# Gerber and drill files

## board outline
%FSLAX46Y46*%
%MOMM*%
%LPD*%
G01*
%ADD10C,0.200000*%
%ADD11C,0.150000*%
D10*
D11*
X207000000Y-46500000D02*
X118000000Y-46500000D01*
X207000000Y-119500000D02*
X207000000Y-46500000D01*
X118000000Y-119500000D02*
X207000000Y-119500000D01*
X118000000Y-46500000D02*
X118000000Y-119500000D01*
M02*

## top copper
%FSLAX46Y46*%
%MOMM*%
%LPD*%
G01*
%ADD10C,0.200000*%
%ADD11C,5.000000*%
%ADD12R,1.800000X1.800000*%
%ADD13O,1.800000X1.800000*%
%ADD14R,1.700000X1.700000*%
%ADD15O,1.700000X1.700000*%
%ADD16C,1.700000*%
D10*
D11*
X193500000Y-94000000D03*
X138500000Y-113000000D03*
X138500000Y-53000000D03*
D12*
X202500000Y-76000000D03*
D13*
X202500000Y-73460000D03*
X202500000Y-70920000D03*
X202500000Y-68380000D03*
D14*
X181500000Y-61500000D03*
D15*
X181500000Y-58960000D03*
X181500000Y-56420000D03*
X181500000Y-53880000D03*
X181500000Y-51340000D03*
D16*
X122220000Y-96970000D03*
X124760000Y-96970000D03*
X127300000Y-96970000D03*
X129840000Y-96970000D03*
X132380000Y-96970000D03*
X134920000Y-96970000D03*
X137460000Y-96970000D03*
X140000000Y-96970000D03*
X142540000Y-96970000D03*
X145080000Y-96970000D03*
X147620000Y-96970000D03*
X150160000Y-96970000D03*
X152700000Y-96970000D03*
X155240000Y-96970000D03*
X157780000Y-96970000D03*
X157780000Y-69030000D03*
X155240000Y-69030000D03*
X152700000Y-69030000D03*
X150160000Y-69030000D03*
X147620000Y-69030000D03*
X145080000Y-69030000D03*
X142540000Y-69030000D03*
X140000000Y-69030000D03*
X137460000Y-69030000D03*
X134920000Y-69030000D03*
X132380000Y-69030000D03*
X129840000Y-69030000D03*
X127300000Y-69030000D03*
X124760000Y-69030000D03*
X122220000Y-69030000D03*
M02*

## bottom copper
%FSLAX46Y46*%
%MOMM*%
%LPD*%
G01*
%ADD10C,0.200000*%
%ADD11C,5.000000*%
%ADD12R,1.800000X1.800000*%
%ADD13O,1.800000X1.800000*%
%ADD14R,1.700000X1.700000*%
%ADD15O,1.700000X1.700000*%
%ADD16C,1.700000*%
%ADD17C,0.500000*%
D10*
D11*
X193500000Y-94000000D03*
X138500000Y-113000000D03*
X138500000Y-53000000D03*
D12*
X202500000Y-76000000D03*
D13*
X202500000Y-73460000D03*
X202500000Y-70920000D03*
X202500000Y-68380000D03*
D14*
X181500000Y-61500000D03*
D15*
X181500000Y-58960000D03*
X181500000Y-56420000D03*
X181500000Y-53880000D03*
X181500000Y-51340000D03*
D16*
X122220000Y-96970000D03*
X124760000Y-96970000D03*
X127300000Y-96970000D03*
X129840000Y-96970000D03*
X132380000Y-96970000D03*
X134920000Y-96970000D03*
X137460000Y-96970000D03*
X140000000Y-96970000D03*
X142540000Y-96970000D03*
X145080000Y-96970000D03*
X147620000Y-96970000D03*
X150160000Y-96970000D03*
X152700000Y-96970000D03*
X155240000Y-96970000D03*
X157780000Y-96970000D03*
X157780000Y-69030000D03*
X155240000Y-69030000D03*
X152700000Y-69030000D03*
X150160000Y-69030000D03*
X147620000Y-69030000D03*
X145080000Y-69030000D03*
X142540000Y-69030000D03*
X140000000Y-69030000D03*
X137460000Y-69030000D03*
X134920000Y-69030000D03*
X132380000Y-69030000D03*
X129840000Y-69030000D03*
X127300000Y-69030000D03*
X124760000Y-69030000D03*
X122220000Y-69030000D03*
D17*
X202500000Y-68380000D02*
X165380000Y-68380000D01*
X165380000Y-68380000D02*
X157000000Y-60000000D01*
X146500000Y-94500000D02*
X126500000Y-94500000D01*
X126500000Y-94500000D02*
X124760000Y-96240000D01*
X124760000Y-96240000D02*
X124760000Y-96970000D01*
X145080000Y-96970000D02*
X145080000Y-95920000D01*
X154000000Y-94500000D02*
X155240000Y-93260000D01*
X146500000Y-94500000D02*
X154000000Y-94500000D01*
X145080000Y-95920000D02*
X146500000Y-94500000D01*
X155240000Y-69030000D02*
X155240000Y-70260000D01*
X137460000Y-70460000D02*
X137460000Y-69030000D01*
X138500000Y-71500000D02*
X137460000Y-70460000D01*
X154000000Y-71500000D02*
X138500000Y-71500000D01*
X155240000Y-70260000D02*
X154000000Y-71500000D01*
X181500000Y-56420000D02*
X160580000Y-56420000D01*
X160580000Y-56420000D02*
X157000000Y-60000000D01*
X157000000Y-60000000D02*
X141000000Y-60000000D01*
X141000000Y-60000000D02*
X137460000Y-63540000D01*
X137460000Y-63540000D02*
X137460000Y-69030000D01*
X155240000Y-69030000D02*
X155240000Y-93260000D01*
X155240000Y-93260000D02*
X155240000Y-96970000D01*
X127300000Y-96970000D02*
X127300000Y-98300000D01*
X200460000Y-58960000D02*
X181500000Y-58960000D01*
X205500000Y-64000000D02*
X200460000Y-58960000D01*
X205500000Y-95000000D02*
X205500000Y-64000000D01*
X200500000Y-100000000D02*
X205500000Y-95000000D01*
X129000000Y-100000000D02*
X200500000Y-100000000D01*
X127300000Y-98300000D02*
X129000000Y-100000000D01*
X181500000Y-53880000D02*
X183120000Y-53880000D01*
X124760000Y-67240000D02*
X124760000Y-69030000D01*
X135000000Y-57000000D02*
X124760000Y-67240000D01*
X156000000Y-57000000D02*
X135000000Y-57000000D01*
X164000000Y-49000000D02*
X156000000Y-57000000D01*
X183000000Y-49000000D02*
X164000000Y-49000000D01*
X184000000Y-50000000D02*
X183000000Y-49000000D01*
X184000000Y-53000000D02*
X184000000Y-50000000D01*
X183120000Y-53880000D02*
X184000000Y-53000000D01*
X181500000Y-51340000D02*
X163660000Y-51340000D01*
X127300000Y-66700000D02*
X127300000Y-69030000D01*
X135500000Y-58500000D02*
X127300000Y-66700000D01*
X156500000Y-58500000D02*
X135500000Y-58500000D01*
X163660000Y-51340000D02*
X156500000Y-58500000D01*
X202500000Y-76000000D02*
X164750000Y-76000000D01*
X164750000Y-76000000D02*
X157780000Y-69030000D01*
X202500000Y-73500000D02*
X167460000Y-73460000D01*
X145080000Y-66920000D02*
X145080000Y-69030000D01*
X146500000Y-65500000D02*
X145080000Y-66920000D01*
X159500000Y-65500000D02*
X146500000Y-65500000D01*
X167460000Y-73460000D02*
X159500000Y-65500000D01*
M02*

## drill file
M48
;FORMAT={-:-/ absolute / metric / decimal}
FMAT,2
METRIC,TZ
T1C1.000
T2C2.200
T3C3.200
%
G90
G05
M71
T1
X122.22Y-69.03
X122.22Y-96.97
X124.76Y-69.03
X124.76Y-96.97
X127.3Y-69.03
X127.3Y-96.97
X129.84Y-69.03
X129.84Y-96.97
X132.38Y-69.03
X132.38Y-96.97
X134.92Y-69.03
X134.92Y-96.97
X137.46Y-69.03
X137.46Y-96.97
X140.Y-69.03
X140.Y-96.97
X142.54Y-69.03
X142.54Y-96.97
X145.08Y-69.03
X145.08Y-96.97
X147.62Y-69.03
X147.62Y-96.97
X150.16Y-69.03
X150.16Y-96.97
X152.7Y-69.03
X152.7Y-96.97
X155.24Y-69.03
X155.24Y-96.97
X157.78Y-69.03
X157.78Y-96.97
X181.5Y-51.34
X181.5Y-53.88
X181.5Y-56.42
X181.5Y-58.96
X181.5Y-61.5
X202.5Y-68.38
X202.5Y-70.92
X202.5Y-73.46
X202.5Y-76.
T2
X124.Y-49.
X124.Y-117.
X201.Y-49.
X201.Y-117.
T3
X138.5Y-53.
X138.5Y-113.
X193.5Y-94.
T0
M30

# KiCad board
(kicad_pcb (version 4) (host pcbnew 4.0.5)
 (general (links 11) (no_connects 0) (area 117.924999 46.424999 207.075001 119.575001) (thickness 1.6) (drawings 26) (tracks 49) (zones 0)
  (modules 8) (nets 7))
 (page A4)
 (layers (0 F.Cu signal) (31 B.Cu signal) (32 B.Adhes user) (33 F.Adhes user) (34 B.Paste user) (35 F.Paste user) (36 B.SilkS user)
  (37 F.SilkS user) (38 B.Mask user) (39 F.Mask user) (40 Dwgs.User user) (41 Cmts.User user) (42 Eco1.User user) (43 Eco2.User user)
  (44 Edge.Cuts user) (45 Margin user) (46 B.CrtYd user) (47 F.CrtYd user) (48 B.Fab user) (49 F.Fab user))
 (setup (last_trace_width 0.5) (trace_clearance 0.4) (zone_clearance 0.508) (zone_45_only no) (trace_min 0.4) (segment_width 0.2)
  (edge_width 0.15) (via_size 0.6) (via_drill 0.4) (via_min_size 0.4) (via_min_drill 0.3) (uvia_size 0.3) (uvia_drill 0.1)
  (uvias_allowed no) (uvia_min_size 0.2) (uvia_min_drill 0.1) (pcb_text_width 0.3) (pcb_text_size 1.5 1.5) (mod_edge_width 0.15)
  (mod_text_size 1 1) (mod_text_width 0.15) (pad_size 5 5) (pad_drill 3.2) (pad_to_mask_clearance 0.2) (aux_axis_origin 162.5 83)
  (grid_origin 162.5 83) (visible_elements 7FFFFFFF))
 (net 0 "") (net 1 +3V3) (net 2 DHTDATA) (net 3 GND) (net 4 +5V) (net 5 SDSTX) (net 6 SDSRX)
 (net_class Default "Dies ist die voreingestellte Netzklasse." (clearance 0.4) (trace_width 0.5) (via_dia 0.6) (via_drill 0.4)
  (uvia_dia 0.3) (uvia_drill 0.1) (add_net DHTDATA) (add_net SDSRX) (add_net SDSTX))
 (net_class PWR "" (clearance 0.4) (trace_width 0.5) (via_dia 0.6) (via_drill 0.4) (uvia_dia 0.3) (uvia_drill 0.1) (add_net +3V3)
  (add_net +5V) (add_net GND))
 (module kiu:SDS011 (layer F.Cu) (at 162.5 83 270)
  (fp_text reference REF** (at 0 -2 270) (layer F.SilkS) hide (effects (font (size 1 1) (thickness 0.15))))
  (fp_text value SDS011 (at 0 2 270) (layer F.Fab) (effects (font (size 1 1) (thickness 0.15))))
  (pad "" np_thru_hole circle (at 11 -31 270) (size 5 5) (drill 3.2) (layers *.Cu *.Mask))
  (pad "" np_thru_hole circle (at 30 24 270) (size 5 5) (drill 3.2) (layers *.Cu *.Mask))
  (pad "" np_thru_hole circle (at -30 24 270) (size 5 5) (drill 3.2) (layers *.Cu *.Mask)))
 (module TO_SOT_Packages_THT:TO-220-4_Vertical (layer F.Cu) (at 202.5 76 90)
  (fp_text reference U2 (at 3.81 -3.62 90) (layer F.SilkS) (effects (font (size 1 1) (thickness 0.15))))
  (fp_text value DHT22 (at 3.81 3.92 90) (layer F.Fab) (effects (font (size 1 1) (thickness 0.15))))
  (pad 1 thru_hole rect (at 0 0 90) (size 1.8 1.8) (drill 1) (layers *.Cu *.Mask) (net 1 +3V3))
  (pad 2 thru_hole oval (at 2.54 0 90) (size 1.8 1.8) (drill 1) (layers *.Cu *.Mask) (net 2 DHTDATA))
  (pad 3 thru_hole oval (at 5.08 0 90) (size 1.8 1.8) (drill 1) (layers *.Cu *.Mask))
  (pad 4 thru_hole oval (at 7.62 0 90) (size 1.8 1.8) (drill 1) (layers *.Cu *.Mask) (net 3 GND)))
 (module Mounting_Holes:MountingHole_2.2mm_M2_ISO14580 (layer F.Cu) (at 201 117)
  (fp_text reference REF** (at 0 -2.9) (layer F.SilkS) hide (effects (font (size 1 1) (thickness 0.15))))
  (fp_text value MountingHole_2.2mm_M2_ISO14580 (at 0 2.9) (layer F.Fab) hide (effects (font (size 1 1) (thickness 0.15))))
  (pad 1 np_thru_hole circle (at 0 0) (size 2.2 2.2) (drill 2.2) (layers *.Cu *.Mask)))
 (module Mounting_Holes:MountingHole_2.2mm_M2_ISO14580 (layer F.Cu) (at 201 49)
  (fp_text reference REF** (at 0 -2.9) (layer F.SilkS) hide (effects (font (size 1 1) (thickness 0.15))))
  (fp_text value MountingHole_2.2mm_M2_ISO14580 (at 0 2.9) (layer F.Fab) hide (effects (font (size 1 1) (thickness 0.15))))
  (pad 1 np_thru_hole circle (at 0 0) (size 2.2 2.2) (drill 2.2) (layers *.Cu *.Mask)))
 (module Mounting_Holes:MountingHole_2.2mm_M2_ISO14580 (layer F.Cu) (at 124 49)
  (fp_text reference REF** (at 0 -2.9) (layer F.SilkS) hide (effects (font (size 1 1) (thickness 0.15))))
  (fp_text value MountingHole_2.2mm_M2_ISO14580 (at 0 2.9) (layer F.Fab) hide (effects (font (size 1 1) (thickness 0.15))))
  (pad 1 np_thru_hole circle (at 0 0) (size 2.2 2.2) (drill 2.2) (layers *.Cu *.Mask)))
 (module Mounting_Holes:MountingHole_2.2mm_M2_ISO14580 (layer F.Cu) (at 124 117)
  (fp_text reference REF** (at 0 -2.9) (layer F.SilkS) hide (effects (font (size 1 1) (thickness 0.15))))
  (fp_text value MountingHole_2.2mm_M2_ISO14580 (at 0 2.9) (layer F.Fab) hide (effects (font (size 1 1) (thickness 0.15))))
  (pad 1 np_thru_hole circle (at 0 0) (size 2.2 2.2) (drill 2.2) (layers *.Cu *.Mask)))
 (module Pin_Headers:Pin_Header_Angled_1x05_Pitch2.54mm (layer F.Cu) (at 181.5 61.5 180)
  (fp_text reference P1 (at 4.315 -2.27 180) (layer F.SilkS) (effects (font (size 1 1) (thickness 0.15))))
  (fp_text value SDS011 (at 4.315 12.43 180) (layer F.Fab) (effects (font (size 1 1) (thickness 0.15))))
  (pad 1 thru_hole rect (at 0 0 180) (size 1.7 1.7) (drill 1) (layers *.Cu *.Mask))
  (pad 2 thru_hole oval (at 0 2.54 180) (size 1.7 1.7) (drill 1) (layers *.Cu *.Mask) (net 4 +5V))
  (pad 3 thru_hole oval (at 0 5.08 180) (size 1.7 1.7) (drill 1) (layers *.Cu *.Mask) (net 3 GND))
  (pad 4 thru_hole oval (at 0 7.62 180) (size 1.7 1.7) (drill 1) (layers *.Cu *.Mask) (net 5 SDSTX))
  (pad 5 thru_hole oval (at 0 10.16 180) (size 1.7 1.7) (drill 1) (layers *.Cu *.Mask) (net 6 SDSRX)))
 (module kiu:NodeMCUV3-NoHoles (layer F.Cu) (at 140 83 90)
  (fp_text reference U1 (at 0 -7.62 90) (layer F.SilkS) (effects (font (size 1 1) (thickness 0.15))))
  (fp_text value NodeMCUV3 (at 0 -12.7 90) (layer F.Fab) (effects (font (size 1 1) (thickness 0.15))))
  (pad 1 thru_hole circle (at -13.97 -17.78 90) (size 1.7 1.7) (drill 1) (layers *.Cu *.Mask))
  (pad 2 thru_hole circle (at -13.97 -15.24 90) (size 1.7 1.7) (drill 1) (layers *.Cu *.Mask) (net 3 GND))
  (pad 3 thru_hole circle (at -13.97 -12.7 90) (size 1.7 1.7) (drill 1) (layers *.Cu *.Mask) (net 4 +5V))
  (pad 4 thru_hole circle (at -13.97 -10.16 90) (size 1.7 1.7) (drill 1) (layers *.Cu *.Mask))
  (pad 5 thru_hole circle (at -13.97 -7.62 90) (size 1.7 1.7) (drill 1) (layers *.Cu *.Mask))
  (pad 6 thru_hole circle (at -13.97 -5.08 90) (size 1.7 1.7) (drill 1) (layers *.Cu *.Mask))
  (pad 7 thru_hole circle (at -13.97 -2.54 90) (size 1.7 1.7) (drill 1) (layers *.Cu *.Mask))
  (pad 8 thru_hole circle (at -13.97 0 90) (size 1.7 1.7) (drill 1) (layers *.Cu *.Mask))
  (pad 9 thru_hole circle (at -13.97 2.54 90) (size 1.7 1.7) (drill 1) (layers *.Cu *.Mask))
  (pad 10 thru_hole circle (at -13.97 5.08 90) (size 1.7 1.7) (drill 1) (layers *.Cu *.Mask) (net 3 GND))
  (pad 11 thru_hole circle (at -13.97 7.62 90) (size 1.7 1.7) (drill 1) (layers *.Cu *.Mask))
  (pad 12 thru_hole circle (at -13.97 10.16 90) (size 1.7 1.7) (drill 1) (layers *.Cu *.Mask))
  (pad 13 thru_hole circle (at -13.97 12.7 90) (size 1.7 1.7) (drill 1) (layers *.Cu *.Mask))
  (pad 14 thru_hole circle (at -13.97 15.24 90) (size 1.7 1.7) (drill 1) (layers *.Cu *.Mask) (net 3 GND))
  (pad 15 thru_hole circle (at -13.97 17.78 90) (size 1.7 1.7) (drill 1) (layers *.Cu *.Mask))
  (pad 16 thru_hole circle (at 13.97 17.78 90) (size 1.7 1.7) (drill 1) (layers *.Cu *.Mask) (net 1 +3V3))
  (pad 17 thru_hole circle (at 13.97 15.24 90) (size 1.7 1.7) (drill 1) (layers *.Cu *.Mask) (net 3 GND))
  (pad 18 thru_hole circle (at 13.97 12.7 90) (size 1.7 1.7) (drill 1) (layers *.Cu *.Mask))
  (pad 19 thru_hole circle (at 13.97 10.16 90) (size 1.7 1.7) (drill 1) (layers *.Cu *.Mask))
  (pad 20 thru_hole circle (at 13.97 7.62 90) (size 1.7 1.7) (drill 1) (layers *.Cu *.Mask))
  (pad 21 thru_hole circle (at 13.97 5.08 90) (size 1.7 1.7) (drill 1) (layers *.Cu *.Mask) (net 2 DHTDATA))
  (pad 22 thru_hole circle (at 13.97 2.54 90) (size 1.7 1.7) (drill 1) (layers *.Cu *.Mask))
  (pad 23 thru_hole circle (at 13.97 0 90) (size 1.7 1.7) (drill 1) (layers *.Cu *.Mask))
  (pad 24 thru_hole circle (at 13.97 -2.54 90) (size 1.7 1.7) (drill 1) (layers *.Cu *.Mask) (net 3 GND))
  (pad 25 thru_hole circle (at 13.97 -5.08 90) (size 1.7 1.7) (drill 1) (layers *.Cu *.Mask))
  (pad 26 thru_hole circle (at 13.97 -7.62 90) (size 1.7 1.7) (drill 1) (layers *.Cu *.Mask))
  (pad 27 thru_hole circle (at 13.97 -10.16 90) (size 1.7 1.7) (drill 1) (layers *.Cu *.Mask))
  (pad 28 thru_hole circle (at 13.97 -12.7 90) (size 1.7 1.7) (drill 1) (layers *.Cu *.Mask) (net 6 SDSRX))
  (pad 29 thru_hole circle (at 13.97 -15.24 90) (size 1.7 1.7) (drill 1) (layers *.Cu *.Mask) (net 5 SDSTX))
  (pad 30 thru_hole circle (at 13.97 -17.78 90) (size 1.7 1.7) (drill 1) (layers *.Cu *.Mask)))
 (gr_line (start 207 46.5) (end 118 46.5) (angle 90) (layer Edge.Cuts) (width 0.15))
 (gr_line (start 207 119.5) (end 207 46.5) (angle 90) (layer Edge.Cuts) (width 0.15))
 (gr_line (start 118 119.5) (end 207 119.5) (angle 90) (layer Edge.Cuts) (width 0.15))
 (gr_line (start 118 46.5) (end 118 119.5) (angle 90) (layer Edge.Cuts) (width 0.15))
 (segment (start 202.5 68.38) (end 165.38 68.38) (width 0.5) (layer B.Cu) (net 3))
 (segment (start 165.38 68.38) (end 157 60) (width 0.5) (layer B.Cu) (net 3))
 (segment (start 146.5 94.5) (end 126.5 94.5) (width 0.5) (layer B.Cu) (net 3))
 (segment (start 126.5 94.5) (end 124.76 96.24) (width 0.5) (layer B.Cu) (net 3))
 (segment (start 124.76 96.24) (end 124.76 96.97) (width 0.5) (layer B.Cu) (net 3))
 (segment (start 145.08 96.97) (end 145.08 95.92) (width 0.5) (layer B.Cu) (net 3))
 (segment (start 154 94.5) (end 155.24 93.26) (width 0.5) (layer B.Cu) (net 3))
 (segment (start 146.5 94.5) (end 154 94.5) (width 0.5) (layer B.Cu) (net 3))
 (segment (start 145.08 95.92) (end 146.5 94.5) (width 0.5) (layer B.Cu) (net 3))
 (segment (start 155.24 69.03) (end 155.24 70.26) (width 0.5) (layer B.Cu) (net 3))
 (segment (start 137.46 70.46) (end 137.46 69.03) (width 0.5) (layer B.Cu) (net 3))
 (segment (start 138.5 71.5) (end 137.46 70.46) (width 0.5) (layer B.Cu) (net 3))
 (segment (start 154 71.5) (end 138.5 71.5) (width 0.5) (layer B.Cu) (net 3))
 (segment (start 155.24 70.26) (end 154 71.5) (width 0.5) (layer B.Cu) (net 3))
 (segment (start 181.5 56.42) (end 160.58 56.42) (width 0.5) (layer B.Cu) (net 3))
 (segment (start 160.58 56.42) (end 157 60) (width 0.5) (layer B.Cu) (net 3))
 (segment (start 157 60) (end 141 60) (width 0.5) (layer B.Cu) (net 3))
 (segment (start 141 60) (end 137.46 63.54) (width 0.5) (layer B.Cu) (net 3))
 (segment (start 137.46 63.54) (end 137.46 69.03) (width 0.5) (layer B.Cu) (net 3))
 (segment (start 155.24 69.03) (end 155.24 93.26) (width 0.5) (layer B.Cu) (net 3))
 (segment (start 155.24 93.26) (end 155.24 96.97) (width 0.5) (layer B.Cu) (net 3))
 (segment (start 127.3 96.97) (end 127.3 98.3) (width 0.5) (layer B.Cu) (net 4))
 (segment (start 200.46 58.96) (end 181.5 58.96) (width 0.5) (layer B.Cu) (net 4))
 (segment (start 205.5 64) (end 200.46 58.96) (width 0.5) (layer B.Cu) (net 4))
 (segment (start 205.5 95) (end 205.5 64) (width 0.5) (layer B.Cu) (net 4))
 (segment (start 200.5 100) (end 205.5 95) (width 0.5) (layer B.Cu) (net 4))
 (segment (start 129 100) (end 200.5 100) (width 0.5) (layer B.Cu) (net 4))
 (segment (start 127.3 98.3) (end 129 100) (width 0.5) (layer B.Cu) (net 4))
 (segment (start 181.5 53.88) (end 183.12 53.88) (width 0.5) (layer B.Cu) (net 5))
 (segment (start 124.76 67.24) (end 124.76 69.03) (width 0.5) (layer B.Cu) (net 5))
 (segment (start 135 57) (end 124.76 67.24) (width 0.5) (layer B.Cu) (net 5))
 (segment (start 156 57) (end 135 57) (width 0.5) (layer B.Cu) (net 5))
 (segment (start 164 49) (end 156 57) (width 0.5) (layer B.Cu) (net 5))
 (segment (start 183 49) (end 164 49) (width 0.5) (layer B.Cu) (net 5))
 (segment (start 184 50) (end 183 49) (width 0.5) (layer B.Cu) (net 5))
 (segment (start 184 53) (end 184 50) (width 0.5) (layer B.Cu) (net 5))
 (segment (start 183.12 53.88) (end 184 53) (width 0.5) (layer B.Cu) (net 5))
 (segment (start 181.5 51.34) (end 163.66 51.34) (width 0.5) (layer B.Cu) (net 6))
 (segment (start 127.3 66.7) (end 127.3 69.03) (width 0.5) (layer B.Cu) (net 6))
 (segment (start 135.5 58.5) (end 127.3 66.7) (width 0.5) (layer B.Cu) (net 6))
 (segment (start 156.5 58.5) (end 135.5 58.5) (width 0.5) (layer B.Cu) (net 6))
 (segment (start 163.66 51.34) (end 156.5 58.5) (width 0.5) (layer B.Cu) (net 6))
 (segment (start 202.5 76) (end 164.75 76) (width 0.5) (layer B.Cu) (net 1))
 (segment (start 164.75 76) (end 157.78 69.03) (width 0.5) (layer B.Cu) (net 1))
 (segment (start 202.5 73.5) (end 167.46 73.46) (width 0.5) (layer B.Cu) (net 2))
 (segment (start 145.08 66.92) (end 145.08 69.03) (width 0.5) (layer B.Cu) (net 2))
 (segment (start 146.5 65.5) (end 145.08 66.92) (width 0.5) (layer B.Cu) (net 2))
 (segment (start 159.5 65.5) (end 146.5 65.5) (width 0.5) (layer B.Cu) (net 2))
 (segment (start 167.46 73.46) (end 159.5 65.5) (width 0.5) (layer B.Cu) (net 2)))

